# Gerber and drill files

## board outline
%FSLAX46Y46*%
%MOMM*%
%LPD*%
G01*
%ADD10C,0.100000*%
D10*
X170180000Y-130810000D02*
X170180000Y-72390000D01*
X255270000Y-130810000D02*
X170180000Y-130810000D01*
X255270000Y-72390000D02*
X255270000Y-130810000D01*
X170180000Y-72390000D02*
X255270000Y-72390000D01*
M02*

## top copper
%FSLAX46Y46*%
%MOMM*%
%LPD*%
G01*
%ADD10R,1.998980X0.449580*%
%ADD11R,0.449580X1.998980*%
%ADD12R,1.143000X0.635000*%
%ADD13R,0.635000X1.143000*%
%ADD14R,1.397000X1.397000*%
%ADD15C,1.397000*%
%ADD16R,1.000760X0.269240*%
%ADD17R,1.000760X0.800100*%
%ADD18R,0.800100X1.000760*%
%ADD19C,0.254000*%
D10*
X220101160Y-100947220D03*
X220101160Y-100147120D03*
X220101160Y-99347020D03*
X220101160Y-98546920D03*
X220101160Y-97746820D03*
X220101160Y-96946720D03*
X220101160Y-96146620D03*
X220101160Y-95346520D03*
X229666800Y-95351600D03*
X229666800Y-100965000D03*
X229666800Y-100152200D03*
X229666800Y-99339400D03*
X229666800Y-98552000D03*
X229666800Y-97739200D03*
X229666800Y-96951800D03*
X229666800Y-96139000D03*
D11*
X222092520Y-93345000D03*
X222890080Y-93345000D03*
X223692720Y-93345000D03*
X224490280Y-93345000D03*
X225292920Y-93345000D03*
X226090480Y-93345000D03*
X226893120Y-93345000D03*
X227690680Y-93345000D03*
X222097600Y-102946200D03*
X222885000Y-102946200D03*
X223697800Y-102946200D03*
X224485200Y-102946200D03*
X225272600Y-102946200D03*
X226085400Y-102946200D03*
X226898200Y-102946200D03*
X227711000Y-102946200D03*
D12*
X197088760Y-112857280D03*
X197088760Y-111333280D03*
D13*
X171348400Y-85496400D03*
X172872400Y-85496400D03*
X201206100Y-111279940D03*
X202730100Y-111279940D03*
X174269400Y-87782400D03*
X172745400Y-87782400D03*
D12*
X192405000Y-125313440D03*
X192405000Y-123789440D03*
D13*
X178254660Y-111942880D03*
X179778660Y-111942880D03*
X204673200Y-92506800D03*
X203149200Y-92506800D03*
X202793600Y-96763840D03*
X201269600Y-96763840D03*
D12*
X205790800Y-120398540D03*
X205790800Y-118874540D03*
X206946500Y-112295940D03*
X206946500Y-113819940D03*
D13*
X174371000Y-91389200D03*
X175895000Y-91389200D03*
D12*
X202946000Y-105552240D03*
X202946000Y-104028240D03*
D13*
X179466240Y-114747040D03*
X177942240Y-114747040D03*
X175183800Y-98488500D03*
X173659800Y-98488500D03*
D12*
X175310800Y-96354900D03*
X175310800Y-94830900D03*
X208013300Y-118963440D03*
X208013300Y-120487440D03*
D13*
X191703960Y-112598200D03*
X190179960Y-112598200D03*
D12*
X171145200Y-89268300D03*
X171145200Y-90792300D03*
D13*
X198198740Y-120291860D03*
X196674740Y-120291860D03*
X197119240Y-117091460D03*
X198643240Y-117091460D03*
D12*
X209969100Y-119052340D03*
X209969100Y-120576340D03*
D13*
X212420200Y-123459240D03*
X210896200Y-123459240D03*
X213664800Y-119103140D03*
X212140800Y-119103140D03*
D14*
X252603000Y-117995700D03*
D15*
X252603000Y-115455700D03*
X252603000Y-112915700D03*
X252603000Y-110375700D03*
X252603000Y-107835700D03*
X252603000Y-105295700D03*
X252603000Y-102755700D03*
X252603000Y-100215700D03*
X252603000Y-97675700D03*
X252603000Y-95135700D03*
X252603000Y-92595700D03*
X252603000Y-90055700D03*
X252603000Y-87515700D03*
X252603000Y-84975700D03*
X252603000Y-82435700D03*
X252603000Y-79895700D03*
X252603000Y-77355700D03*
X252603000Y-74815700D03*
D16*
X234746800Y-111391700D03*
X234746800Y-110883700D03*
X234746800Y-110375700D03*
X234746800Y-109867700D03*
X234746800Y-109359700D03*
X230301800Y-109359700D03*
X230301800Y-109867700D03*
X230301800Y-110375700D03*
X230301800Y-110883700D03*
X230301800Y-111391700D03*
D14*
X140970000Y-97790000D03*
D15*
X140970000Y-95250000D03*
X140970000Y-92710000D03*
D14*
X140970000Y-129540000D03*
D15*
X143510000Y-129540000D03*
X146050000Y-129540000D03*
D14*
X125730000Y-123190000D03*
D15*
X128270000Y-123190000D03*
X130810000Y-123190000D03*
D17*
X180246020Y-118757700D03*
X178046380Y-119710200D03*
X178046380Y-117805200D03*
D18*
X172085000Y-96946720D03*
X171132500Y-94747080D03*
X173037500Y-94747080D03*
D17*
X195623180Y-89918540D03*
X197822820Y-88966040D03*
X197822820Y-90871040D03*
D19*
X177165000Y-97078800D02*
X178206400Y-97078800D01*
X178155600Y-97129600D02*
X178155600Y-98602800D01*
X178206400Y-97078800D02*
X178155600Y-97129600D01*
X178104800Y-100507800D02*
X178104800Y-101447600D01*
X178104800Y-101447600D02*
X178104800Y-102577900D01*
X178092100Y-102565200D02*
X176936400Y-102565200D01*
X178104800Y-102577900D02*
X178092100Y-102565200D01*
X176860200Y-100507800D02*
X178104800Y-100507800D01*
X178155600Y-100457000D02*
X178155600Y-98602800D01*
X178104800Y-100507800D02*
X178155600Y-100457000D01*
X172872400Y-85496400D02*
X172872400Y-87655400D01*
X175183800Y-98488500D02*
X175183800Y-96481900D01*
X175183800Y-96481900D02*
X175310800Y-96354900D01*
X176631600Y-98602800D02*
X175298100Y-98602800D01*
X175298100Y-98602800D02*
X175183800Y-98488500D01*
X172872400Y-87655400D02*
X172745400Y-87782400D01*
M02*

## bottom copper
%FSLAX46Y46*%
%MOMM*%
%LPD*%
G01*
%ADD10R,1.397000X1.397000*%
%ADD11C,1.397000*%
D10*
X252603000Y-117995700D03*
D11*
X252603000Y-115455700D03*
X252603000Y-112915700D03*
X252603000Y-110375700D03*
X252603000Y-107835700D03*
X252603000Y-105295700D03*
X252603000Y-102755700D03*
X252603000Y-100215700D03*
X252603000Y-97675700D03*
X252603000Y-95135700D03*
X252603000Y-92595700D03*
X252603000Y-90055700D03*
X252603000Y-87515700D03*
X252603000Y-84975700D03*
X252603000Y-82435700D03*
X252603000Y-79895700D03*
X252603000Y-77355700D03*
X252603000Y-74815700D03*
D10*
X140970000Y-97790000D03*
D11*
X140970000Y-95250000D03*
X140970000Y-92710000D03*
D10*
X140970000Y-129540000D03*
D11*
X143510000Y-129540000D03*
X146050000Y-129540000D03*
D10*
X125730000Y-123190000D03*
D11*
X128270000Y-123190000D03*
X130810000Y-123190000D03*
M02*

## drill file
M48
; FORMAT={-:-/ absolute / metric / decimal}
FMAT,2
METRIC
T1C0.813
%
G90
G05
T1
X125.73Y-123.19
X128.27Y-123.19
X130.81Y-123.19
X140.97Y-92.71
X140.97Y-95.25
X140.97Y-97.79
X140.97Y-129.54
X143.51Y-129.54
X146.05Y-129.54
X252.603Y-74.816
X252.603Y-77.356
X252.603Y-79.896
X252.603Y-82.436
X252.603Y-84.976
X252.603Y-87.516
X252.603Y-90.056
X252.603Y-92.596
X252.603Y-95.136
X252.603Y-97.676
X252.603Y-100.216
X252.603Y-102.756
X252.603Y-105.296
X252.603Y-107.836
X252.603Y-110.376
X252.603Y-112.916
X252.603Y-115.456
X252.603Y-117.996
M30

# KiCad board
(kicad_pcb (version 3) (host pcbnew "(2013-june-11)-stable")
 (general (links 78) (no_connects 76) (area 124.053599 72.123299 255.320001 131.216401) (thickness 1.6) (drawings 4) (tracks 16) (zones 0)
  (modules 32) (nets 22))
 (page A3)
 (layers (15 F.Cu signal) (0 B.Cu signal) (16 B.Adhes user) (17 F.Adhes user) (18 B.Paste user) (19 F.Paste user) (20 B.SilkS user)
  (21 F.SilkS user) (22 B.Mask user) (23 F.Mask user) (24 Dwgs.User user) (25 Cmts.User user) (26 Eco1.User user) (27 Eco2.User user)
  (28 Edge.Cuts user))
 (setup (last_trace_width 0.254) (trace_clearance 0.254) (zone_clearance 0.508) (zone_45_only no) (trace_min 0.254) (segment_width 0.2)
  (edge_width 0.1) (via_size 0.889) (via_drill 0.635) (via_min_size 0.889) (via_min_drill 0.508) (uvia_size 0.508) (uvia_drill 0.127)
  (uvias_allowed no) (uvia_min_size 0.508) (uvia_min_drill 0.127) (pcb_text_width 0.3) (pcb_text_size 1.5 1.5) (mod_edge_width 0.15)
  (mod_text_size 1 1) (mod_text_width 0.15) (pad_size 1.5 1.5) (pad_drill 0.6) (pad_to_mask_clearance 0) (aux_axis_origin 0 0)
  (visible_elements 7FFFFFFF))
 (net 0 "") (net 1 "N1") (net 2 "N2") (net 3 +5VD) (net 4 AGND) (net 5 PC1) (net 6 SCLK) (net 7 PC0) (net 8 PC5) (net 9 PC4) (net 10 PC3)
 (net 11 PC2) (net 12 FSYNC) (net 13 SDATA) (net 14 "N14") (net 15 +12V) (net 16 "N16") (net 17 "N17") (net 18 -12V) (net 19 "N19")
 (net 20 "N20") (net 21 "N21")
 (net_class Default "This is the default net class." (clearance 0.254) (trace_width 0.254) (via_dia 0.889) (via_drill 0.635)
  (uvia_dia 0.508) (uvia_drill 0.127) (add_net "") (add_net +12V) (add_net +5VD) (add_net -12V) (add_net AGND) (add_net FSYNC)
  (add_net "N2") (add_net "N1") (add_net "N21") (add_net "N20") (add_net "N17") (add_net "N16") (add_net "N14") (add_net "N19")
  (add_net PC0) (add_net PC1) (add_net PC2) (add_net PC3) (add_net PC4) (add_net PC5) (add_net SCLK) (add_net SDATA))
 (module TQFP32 (layer F.Cu) (at 224.917 98.171)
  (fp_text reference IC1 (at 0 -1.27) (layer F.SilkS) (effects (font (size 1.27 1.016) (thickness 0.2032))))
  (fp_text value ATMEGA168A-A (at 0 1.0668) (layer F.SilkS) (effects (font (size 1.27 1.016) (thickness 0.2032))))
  (pad 8 smd rect (at -4.81584 2.77622) (size 1.99898 0.44958) (layers F.Cu F.Paste F.Mask) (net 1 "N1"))
  (pad 7 smd rect (at -4.81584 1.97612) (size 1.99898 0.44958) (layers F.Cu F.Paste F.Mask) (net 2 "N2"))
  (pad 6 smd rect (at -4.81584 1.17602) (size 1.99898 0.44958) (layers F.Cu F.Paste F.Mask) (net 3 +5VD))
  (pad 5 smd rect (at -4.81584 0.37592) (size 1.99898 0.44958) (layers F.Cu F.Paste F.Mask) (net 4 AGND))
  (pad 4 smd rect (at -4.81584 -0.42418) (size 1.99898 0.44958) (layers F.Cu F.Paste F.Mask) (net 3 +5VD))
  (pad 3 smd rect (at -4.81584 -1.22428) (size 1.99898 0.44958) (layers F.Cu F.Paste F.Mask) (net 4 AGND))
  (pad 2 smd rect (at -4.81584 -2.02438) (size 1.99898 0.44958) (layers F.Cu F.Paste F.Mask))
  (pad 1 smd rect (at -4.81584 -2.82448) (size 1.99898 0.44958) (layers F.Cu F.Paste F.Mask))
  (pad 24 smd rect (at 4.7498 -2.8194) (size 1.99898 0.44958) (layers F.Cu F.Paste F.Mask) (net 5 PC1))
  (pad 17 smd rect (at 4.7498 2.794) (size 1.99898 0.44958) (layers F.Cu F.Paste F.Mask) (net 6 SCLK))
  (pad 18 smd rect (at 4.7498 1.9812) (size 1.99898 0.44958) (layers F.Cu F.Paste F.Mask) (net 3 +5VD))
  (pad 19 smd rect (at 4.7498 1.1684) (size 1.99898 0.44958) (layers F.Cu F.Paste F.Mask))
  (pad 20 smd rect (at 4.7498 0.381) (size 1.99898 0.44958) (layers F.Cu F.Paste F.Mask))
  (pad 21 smd rect (at 4.7498 -0.4318) (size 1.99898 0.44958) (layers F.Cu F.Paste F.Mask) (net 4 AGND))
  (pad 22 smd rect (at 4.7498 -1.2192) (size 1.99898 0.44958) (layers F.Cu F.Paste F.Mask))
  (pad 23 smd rect (at 4.7498 -2.032) (size 1.99898 0.44958) (layers F.Cu F.Paste F.Mask) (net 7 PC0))
  (pad 32 smd rect (at -2.82448 -4.826) (size 0.44958 1.99898) (layers F.Cu F.Paste F.Mask))
  (pad 31 smd rect (at -2.02692 -4.826) (size 0.44958 1.99898) (layers F.Cu F.Paste F.Mask))
  (pad 30 smd rect (at -1.22428 -4.826) (size 0.44958 1.99898) (layers F.Cu F.Paste F.Mask))
  (pad 29 smd rect (at -0.42672 -4.826) (size 0.44958 1.99898) (layers F.Cu F.Paste F.Mask))
  (pad 28 smd rect (at 0.37592 -4.826) (size 0.44958 1.99898) (layers F.Cu F.Paste F.Mask) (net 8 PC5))
  (pad 27 smd rect (at 1.17348 -4.826) (size 0.44958 1.99898) (layers F.Cu F.Paste F.Mask) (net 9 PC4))
  (pad 26 smd rect (at 1.97612 -4.826) (size 0.44958 1.99898) (layers F.Cu F.Paste F.Mask) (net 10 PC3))
  (pad 25 smd rect (at 2.77368 -4.826) (size 0.44958 1.99898) (layers F.Cu F.Paste F.Mask) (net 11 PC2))
  (pad 9 smd rect (at -2.8194 4.7752) (size 0.44958 1.99898) (layers F.Cu F.Paste F.Mask))
  (pad 10 smd rect (at -2.032 4.7752) (size 0.44958 1.99898) (layers F.Cu F.Paste F.Mask))
  (pad 11 smd rect (at -1.2192 4.7752) (size 0.44958 1.99898) (layers F.Cu F.Paste F.Mask))
  (pad 12 smd rect (at -0.4318 4.7752) (size 0.44958 1.99898) (layers F.Cu F.Paste F.Mask))
  (pad 13 smd rect (at 0.3556 4.7752) (size 0.44958 1.99898) (layers F.Cu F.Paste F.Mask))
  (pad 14 smd rect (at 1.1684 4.7752) (size 0.44958 1.99898) (layers F.Cu F.Paste F.Mask))
  (pad 15 smd rect (at 1.9812 4.7752) (size 0.44958 1.99898) (layers F.Cu F.Paste F.Mask) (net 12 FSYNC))
  (pad 16 smd rect (at 2.794 4.7752) (size 0.44958 1.99898) (layers F.Cu F.Paste F.Mask) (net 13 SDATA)))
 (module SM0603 (layer F.Cu) (at 197.08876 112.09528 90)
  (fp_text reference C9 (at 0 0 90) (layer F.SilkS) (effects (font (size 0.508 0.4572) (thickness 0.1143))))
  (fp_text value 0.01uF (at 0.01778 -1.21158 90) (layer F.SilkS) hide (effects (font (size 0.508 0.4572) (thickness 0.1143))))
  (pad 1 smd rect (at -0.762 0 90) (size 0.635 1.143) (layers F.Cu F.Paste F.Mask) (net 4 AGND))
  (pad 2 smd rect (at 0.762 0 90) (size 0.635 1.143) (layers F.Cu F.Paste F.Mask) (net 3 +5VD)))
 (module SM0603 (layer F.Cu) (at 172.1104 85.4964)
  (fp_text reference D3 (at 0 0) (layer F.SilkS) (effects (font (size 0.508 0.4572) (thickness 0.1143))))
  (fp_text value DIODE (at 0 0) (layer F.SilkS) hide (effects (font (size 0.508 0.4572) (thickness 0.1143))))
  (pad 1 smd rect (at -0.762 0) (size 0.635 1.143) (layers F.Cu F.Paste F.Mask) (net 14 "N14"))
  (pad 2 smd rect (at 0.762 0) (size 0.635 1.143) (layers F.Cu F.Paste F.Mask) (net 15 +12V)))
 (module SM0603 (layer F.Cu) (at 201.9681 111.27994)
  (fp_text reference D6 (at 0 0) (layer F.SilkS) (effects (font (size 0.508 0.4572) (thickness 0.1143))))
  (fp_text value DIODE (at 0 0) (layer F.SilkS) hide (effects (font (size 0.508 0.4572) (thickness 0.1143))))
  (pad 1 smd rect (at -0.762 0) (size 0.635 1.143) (layers F.Cu F.Paste F.Mask) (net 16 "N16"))
  (pad 2 smd rect (at 0.762 0) (size 0.635 1.143) (layers F.Cu F.Paste F.Mask) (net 3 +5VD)))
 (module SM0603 (layer F.Cu) (at 173.5074 87.7824 180)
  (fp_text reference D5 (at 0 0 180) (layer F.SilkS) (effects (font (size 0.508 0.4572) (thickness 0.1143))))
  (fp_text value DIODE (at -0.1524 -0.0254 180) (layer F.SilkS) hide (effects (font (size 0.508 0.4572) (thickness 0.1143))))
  (pad 1 smd rect (at -0.762 0 180) (size 0.635 1.143) (layers F.Cu F.Paste F.Mask) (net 3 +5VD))
  (pad 2 smd rect (at 0.762 0 180) (size 0.635 1.143) (layers F.Cu F.Paste F.Mask) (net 15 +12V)))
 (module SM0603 (layer F.Cu) (at 192.405 124.55144 90)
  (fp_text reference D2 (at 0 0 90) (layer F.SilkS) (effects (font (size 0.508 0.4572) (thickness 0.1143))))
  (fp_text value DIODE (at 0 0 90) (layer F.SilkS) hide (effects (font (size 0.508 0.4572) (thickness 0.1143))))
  (pad 1 smd rect (at -0.762 0 90) (size 0.635 1.143) (layers F.Cu F.Paste F.Mask))
  (pad 2 smd rect (at 0.762 0 90) (size 0.635 1.143) (layers F.Cu F.Paste F.Mask)))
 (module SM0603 (layer F.Cu) (at 179.01666 111.94288)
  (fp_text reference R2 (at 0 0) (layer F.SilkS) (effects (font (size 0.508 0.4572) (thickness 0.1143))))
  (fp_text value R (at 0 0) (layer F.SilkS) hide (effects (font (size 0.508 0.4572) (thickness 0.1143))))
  (pad 1 smd rect (at -0.762 0) (size 0.635 1.143) (layers F.Cu F.Paste F.Mask) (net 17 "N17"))
  (pad 2 smd rect (at 0.762 0) (size 0.635 1.143) (layers F.Cu F.Paste F.Mask) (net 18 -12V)))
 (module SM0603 (layer F.Cu) (at 203.9112 92.5068 180)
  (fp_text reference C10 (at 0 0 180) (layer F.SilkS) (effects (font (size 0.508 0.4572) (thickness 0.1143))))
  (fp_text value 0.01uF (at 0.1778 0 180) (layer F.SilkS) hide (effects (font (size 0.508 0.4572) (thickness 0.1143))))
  (pad 1 smd rect (at -0.762 0 180) (size 0.635 1.143) (layers F.Cu F.Paste F.Mask) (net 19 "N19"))
  (pad 2 smd rect (at 0.762 0 180) (size 0.635 1.143) (layers F.Cu F.Paste F.Mask) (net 3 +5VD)))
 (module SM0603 (layer F.Cu) (at 202.0316 96.76384 180)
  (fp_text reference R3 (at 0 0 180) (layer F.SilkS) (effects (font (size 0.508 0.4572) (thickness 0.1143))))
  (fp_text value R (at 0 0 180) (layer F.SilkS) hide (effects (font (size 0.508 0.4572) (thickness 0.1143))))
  (pad 1 smd rect (at -0.762 0 180) (size 0.635 1.143) (layers F.Cu F.Paste F.Mask) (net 3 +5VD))
  (pad 2 smd rect (at 0.762 0 180) (size 0.635 1.143) (layers F.Cu F.Paste F.Mask) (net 16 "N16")))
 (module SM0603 (layer F.Cu) (at 205.7908 119.63654 90)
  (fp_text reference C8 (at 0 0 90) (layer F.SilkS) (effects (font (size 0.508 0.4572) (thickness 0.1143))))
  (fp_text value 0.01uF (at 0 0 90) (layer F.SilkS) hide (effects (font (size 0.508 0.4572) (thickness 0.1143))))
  (pad 1 smd rect (at -0.762 0 90) (size 0.635 1.143) (layers F.Cu F.Paste F.Mask) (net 4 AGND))
  (pad 2 smd rect (at 0.762 0 90) (size 0.635 1.143) (layers F.Cu F.Paste F.Mask) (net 3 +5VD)))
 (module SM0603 (layer F.Cu) (at 206.9465 113.05794 270)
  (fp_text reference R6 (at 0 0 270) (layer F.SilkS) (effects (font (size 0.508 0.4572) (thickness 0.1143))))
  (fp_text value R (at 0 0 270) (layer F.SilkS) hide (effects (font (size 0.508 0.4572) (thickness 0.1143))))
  (pad 1 smd rect (at -0.762 0 270) (size 0.635 1.143) (layers F.Cu F.Paste F.Mask) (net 3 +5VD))
  (pad 2 smd rect (at 0.762 0 270) (size 0.635 1.143) (layers F.Cu F.Paste F.Mask) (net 12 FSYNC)))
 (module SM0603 (layer F.Cu) (at 175.133 91.3892)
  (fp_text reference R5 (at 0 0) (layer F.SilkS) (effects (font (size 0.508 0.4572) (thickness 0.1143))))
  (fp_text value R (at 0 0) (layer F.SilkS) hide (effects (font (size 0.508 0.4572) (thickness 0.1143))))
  (pad 1 smd rect (at -0.762 0) (size 0.635 1.143) (layers F.Cu F.Paste F.Mask) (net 3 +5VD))
  (pad 2 smd rect (at 0.762 0) (size 0.635 1.143) (layers F.Cu F.Paste F.Mask) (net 13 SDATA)))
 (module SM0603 (layer F.Cu) (at 202.946 104.79024 90)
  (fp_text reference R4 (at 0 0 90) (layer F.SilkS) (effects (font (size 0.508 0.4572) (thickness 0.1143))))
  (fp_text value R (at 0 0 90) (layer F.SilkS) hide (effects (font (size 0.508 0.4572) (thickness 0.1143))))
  (pad 1 smd rect (at -0.762 0 90) (size 0.635 1.143) (layers F.Cu F.Paste F.Mask) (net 3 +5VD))
  (pad 2 smd rect (at 0.762 0 90) (size 0.635 1.143) (layers F.Cu F.Paste F.Mask) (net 6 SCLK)))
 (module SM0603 (layer F.Cu) (at 178.70424 114.74704 180)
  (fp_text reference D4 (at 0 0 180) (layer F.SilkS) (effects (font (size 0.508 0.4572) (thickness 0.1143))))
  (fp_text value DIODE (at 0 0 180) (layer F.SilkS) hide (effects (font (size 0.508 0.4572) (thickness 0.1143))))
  (pad 1 smd rect (at -0.762 0 180) (size 0.635 1.143) (layers F.Cu F.Paste F.Mask) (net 18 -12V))
  (pad 2 smd rect (at 0.762 0 180) (size 0.635 1.143) (layers F.Cu F.Paste F.Mask) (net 17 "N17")))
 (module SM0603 (layer F.Cu) (at 174.4218 98.4885 180)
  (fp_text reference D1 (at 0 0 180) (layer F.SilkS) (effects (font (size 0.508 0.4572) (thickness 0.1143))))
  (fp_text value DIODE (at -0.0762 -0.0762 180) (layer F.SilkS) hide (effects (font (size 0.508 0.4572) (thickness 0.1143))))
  (pad 1 smd rect (at -0.762 0 180) (size 0.635 1.143) (layers F.Cu F.Paste F.Mask) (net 15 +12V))
  (pad 2 smd rect (at 0.762 0 180) (size 0.635 1.143) (layers F.Cu F.Paste F.Mask) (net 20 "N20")))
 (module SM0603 (layer F.Cu) (at 175.3108 95.5929 90)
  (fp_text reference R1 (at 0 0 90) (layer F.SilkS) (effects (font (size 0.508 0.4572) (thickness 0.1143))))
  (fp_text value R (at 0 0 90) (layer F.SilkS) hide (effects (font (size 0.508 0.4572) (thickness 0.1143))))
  (pad 1 smd rect (at -0.762 0 90) (size 0.635 1.143) (layers F.Cu F.Paste F.Mask) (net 15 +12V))
  (pad 2 smd rect (at 0.762 0 90) (size 0.635 1.143) (layers F.Cu F.Paste F.Mask) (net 14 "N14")))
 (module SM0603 (layer F.Cu) (at 208.0133 119.72544 270)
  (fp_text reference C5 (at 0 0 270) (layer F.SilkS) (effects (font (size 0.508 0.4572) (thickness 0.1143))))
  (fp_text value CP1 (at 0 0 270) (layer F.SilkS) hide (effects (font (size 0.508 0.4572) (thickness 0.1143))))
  (pad 1 smd rect (at -0.762 0 270) (size 0.635 1.143) (layers F.Cu F.Paste F.Mask) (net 3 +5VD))
  (pad 2 smd rect (at 0.762 0 270) (size 0.635 1.143) (layers F.Cu F.Paste F.Mask) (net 4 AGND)))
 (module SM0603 (layer F.Cu) (at 190.94196 112.5982 180)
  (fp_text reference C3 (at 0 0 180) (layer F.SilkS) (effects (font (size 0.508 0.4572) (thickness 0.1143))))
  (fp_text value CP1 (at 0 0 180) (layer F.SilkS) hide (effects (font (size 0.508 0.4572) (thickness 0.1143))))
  (pad 1 smd rect (at -0.762 0 180) (size 0.635 1.143) (layers F.Cu F.Paste F.Mask) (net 15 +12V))
  (pad 2 smd rect (at 0.762 0 180) (size 0.635 1.143) (layers F.Cu F.Paste F.Mask) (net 4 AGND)))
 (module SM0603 (layer F.Cu) (at 171.1452 90.0303 270)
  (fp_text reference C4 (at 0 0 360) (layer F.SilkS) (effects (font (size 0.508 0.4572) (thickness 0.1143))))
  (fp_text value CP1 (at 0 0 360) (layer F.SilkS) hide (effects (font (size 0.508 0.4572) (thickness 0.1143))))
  (pad 1 smd rect (at -0.762 0 270) (size 0.635 1.143) (layers F.Cu F.Paste F.Mask) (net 4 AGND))
  (pad 2 smd rect (at 0.762 0 270) (size 0.635 1.143) (layers F.Cu F.Paste F.Mask) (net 18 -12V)))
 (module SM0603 (layer F.Cu) (at 197.43674 120.29186 180)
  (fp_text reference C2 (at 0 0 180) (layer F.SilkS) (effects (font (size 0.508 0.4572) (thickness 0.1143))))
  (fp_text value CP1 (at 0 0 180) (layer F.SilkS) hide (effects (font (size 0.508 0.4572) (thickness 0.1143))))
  (pad 1 smd rect (at -0.762 0 180) (size 0.635 1.143) (layers F.Cu F.Paste F.Mask) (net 4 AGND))
  (pad 2 smd rect (at 0.762 0 180) (size 0.635 1.143) (layers F.Cu F.Paste F.Mask) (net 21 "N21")))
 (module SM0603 (layer F.Cu) (at 197.88124 117.09146)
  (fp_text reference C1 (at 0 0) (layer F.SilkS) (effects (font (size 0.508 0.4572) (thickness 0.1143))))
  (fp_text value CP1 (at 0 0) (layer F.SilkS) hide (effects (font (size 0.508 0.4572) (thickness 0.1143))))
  (pad 1 smd rect (at -0.762 0) (size 0.635 1.143) (layers F.Cu F.Paste F.Mask) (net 20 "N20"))
  (pad 2 smd rect (at 0.762 0) (size 0.635 1.143) (layers F.Cu F.Paste F.Mask) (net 4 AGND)))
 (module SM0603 (layer F.Cu) (at 209.9691 119.81434 270)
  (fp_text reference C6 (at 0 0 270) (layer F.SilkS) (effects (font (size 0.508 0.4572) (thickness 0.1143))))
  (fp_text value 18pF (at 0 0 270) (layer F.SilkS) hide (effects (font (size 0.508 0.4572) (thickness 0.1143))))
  (pad 1 smd rect (at -0.762 0 270) (size 0.635 1.143) (layers F.Cu F.Paste F.Mask) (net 2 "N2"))
  (pad 2 smd rect (at 0.762 0 270) (size 0.635 1.143) (layers F.Cu F.Paste F.Mask) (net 4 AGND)))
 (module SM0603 (layer F.Cu) (at 211.6582 123.45924 180)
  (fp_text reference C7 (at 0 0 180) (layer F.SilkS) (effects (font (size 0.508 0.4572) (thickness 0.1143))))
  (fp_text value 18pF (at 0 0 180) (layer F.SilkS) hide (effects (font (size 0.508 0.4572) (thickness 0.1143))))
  (pad 1 smd rect (at -0.762 0 180) (size 0.635 1.143) (layers F.Cu F.Paste F.Mask) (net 1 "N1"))
  (pad 2 smd rect (at 0.762 0 180) (size 0.635 1.143) (layers F.Cu F.Paste F.Mask) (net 4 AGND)))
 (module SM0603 (layer F.Cu) (at 212.9028 119.10314 180)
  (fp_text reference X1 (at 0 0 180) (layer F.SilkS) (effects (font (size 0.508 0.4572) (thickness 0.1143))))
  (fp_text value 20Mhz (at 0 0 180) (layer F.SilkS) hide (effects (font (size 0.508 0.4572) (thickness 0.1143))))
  (pad 1 smd rect (at -0.762 0 180) (size 0.635 1.143) (layers F.Cu F.Paste F.Mask) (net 1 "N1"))
  (pad 2 smd rect (at 0.762 0 180) (size 0.635 1.143) (layers F.Cu F.Paste F.Mask) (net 2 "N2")))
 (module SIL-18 (layer F.Cu) (at 252.603 96.4057 90)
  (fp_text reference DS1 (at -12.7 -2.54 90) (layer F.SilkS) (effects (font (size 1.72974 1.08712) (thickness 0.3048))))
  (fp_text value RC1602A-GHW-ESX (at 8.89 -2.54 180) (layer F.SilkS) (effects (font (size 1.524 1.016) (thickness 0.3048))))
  (pad 1 thru_hole rect (at -21.59 0 90) (size 1.397 1.397) (drill 0.8128) (layers *.Cu *.Mask F.SilkS) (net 4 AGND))
  (pad 2 thru_hole circle (at -19.05 0 90) (size 1.397 1.397) (drill 0.8128) (layers *.Cu *.Mask F.SilkS) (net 3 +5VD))
  (pad 3 thru_hole circle (at -16.51 0 90) (size 1.397 1.397) (drill 0.8128) (layers *.Cu *.Mask F.SilkS) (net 3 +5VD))
  (pad 4 thru_hole circle (at -13.97 0 90) (size 1.397 1.397) (drill 0.8128) (layers *.Cu *.Mask F.SilkS) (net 9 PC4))
  (pad 5 thru_hole circle (at -11.43 0 90) (size 1.397 1.397) (drill 0.8128) (layers *.Cu *.Mask F.SilkS) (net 4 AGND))
  (pad 6 thru_hole circle (at -8.89 0 90) (size 1.397 1.397) (drill 0.8128) (layers *.Cu *.Mask F.SilkS) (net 8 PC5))
  (pad 7 thru_hole circle (at -6.35 0 90) (size 1.397 1.397) (drill 0.8128) (layers *.Cu *.Mask F.SilkS))
  (pad 8 thru_hole circle (at -3.81 0 90) (size 1.397 1.397) (drill 0.8128) (layers *.Cu *.Mask F.SilkS))
  (pad 9 thru_hole circle (at -1.27 0 90) (size 1.397 1.397) (drill 0.8128) (layers *.Cu *.Mask F.SilkS))
  (pad 10 thru_hole circle (at 1.27 0 90) (size 1.397 1.397) (drill 0.8128) (layers *.Cu *.Mask F.SilkS))
  (pad 11 thru_hole circle (at 3.81 0 90) (size 1.397 1.397) (drill 0.8128) (layers *.Cu *.Mask F.SilkS) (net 7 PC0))
  (pad 12 thru_hole circle (at 6.35 0 90) (size 1.397 1.397) (drill 0.8128) (layers *.Cu *.Mask F.SilkS) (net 5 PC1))
  (pad 13 thru_hole circle (at 8.89 0 90) (size 1.397 1.397) (drill 0.8128) (layers *.Cu *.Mask F.SilkS) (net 11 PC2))
  (pad 14 thru_hole circle (at 11.43 0 90) (size 1.397 1.397) (drill 0.8128) (layers *.Cu *.Mask F.SilkS) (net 10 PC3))
  (pad 15 thru_hole circle (at 13.97 0 90) (size 1.397 1.397) (drill 0.8128) (layers *.Cu *.Mask F.SilkS) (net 3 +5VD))
  (pad 16 thru_hole circle (at 16.51 0 90) (size 1.397 1.397) (drill 0.8128) (layers *.Cu *.Mask F.SilkS) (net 4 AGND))
  (pad 17 thru_hole circle (at 19.05 0 90) (size 1.397 1.397) (drill 0.8128) (layers *.Cu *.Mask F.SilkS))
  (pad 18 thru_hole circle (at 21.59 0 90) (size 1.397 1.397) (drill 0.8128) (layers *.Cu *.Mask F.SilkS)))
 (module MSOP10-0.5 (layer F.Cu) (at 232.5243 110.3757 90)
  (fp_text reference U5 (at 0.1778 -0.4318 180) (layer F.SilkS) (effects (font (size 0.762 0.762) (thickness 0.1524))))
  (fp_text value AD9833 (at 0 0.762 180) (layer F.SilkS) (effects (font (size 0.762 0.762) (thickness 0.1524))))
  (pad 1 smd rect (at -1.016 2.2225 90) (size 0.26924 1.00076) (layers F.Cu F.Paste F.Mask) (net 19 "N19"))
  (pad 2 smd rect (at -0.508 2.2225 90) (size 0.26924 1.00076) (layers F.Cu F.Paste F.Mask) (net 3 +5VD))
  (pad 3 smd rect (at 0 2.2225 90) (size 0.26924 1.00076) (layers F.Cu F.Paste F.Mask) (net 3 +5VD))
  (pad 4 smd rect (at 0.508 2.2225 90) (size 0.26924 1.00076) (layers F.Cu F.Paste F.Mask) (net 4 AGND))
  (pad 5 smd rect (at 1.016 2.2225 90) (size 0.26924 1.00076) (layers F.Cu F.Paste F.Mask))
  (pad 6 smd rect (at 1.016 -2.2225 90) (size 0.26924 1.00076) (layers F.Cu F.Paste F.Mask) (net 13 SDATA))
  (pad 7 smd rect (at 0.508 -2.2225 90) (size 0.26924 1.00076) (layers F.Cu F.Paste F.Mask) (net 6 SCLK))
  (pad 8 smd rect (at 0 -2.2225 90) (size 0.26924 1.00076) (layers F.Cu F.Paste F.Mask) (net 12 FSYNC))
  (pad 9 smd rect (at -0.508 -2.2225 90) (size 0.26924 1.00076) (layers F.Cu F.Paste F.Mask) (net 4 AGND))
  (pad 10 smd rect (at -1.016 -2.2225 90) (size 0.26924 1.00076) (layers F.Cu F.Paste F.Mask)))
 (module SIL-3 (layer F.Cu) (at 140.97 95.25 90)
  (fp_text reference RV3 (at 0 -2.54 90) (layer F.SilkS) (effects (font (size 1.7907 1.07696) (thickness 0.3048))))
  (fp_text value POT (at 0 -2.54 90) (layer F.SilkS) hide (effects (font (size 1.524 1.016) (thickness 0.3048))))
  (pad 1 thru_hole rect (at -2.54 0 90) (size 1.397 1.397) (drill 0.8128) (layers *.Cu *.Mask F.SilkS) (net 16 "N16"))
  (pad 2 thru_hole circle (at 0 0 90) (size 1.397 1.397) (drill 0.8128) (layers *.Cu *.Mask F.SilkS) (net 16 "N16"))
  (pad 3 thru_hole circle (at 2.54 0 90) (size 1.397 1.397) (drill 0.8128) (layers *.Cu *.Mask F.SilkS) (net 4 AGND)))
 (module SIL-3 (layer F.Cu) (at 143.51 129.54)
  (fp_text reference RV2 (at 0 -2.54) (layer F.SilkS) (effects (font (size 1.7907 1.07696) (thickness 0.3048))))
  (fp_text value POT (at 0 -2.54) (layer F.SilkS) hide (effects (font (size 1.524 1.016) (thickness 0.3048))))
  (pad 1 thru_hole rect (at -2.54 0) (size 1.397 1.397) (drill 0.8128) (layers *.Cu *.Mask F.SilkS) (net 4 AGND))
  (pad 2 thru_hole circle (at 0 0) (size 1.397 1.397) (drill 0.8128) (layers *.Cu *.Mask F.SilkS) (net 17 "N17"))
  (pad 3 thru_hole circle (at 2.54 0) (size 1.397 1.397) (drill 0.8128) (layers *.Cu *.Mask F.SilkS) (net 17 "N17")))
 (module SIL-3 (layer F.Cu) (at 128.27 123.19)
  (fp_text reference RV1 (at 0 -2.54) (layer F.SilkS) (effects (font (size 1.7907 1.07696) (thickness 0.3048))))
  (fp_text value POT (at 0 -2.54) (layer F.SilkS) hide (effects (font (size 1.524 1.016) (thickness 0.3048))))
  (pad 1 thru_hole rect (at -2.54 0) (size 1.397 1.397) (drill 0.8128) (layers *.Cu *.Mask F.SilkS) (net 14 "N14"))
  (pad 2 thru_hole circle (at 0 0) (size 1.397 1.397) (drill 0.8128) (layers *.Cu *.Mask F.SilkS) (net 14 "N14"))
  (pad 3 thru_hole circle (at 2.54 0) (size 1.397 1.397) (drill 0.8128) (layers *.Cu *.Mask F.SilkS) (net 4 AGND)))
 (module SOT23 (layer F.Cu) (at 179.1462 118.7577 270)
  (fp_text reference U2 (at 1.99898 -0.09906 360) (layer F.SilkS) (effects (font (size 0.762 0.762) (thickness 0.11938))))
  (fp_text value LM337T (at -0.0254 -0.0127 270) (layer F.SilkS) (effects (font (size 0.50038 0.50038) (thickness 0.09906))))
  (pad 3 smd rect (at 0 -1.09982 270) (size 0.8001 1.00076) (layers F.Cu F.Paste F.Mask) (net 18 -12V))
  (pad 2 smd rect (at 0.9525 1.09982 270) (size 0.8001 1.00076) (layers F.Cu F.Paste F.Mask) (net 21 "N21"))
  (pad 1 smd rect (at -0.9525 1.09982 270) (size 0.8001 1.00076) (layers F.Cu F.Paste F.Mask) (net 17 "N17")))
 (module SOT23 (layer F.Cu) (at 172.085 95.8469 180)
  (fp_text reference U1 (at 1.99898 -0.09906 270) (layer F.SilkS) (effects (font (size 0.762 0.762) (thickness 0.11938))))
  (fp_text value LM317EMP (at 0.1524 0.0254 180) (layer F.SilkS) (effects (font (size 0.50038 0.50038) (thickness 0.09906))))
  (pad 3 smd rect (at 0 -1.09982 180) (size 0.8001 1.00076) (layers F.Cu F.Paste F.Mask) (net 20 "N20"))
  (pad 2 smd rect (at 0.9525 1.09982 180) (size 0.8001 1.00076) (layers F.Cu F.Paste F.Mask) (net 15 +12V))
  (pad 1 smd rect (at -0.9525 1.09982 180) (size 0.8001 1.00076) (layers F.Cu F.Paste F.Mask) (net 14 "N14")))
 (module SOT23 (layer F.Cu) (at 196.723 89.91854 90)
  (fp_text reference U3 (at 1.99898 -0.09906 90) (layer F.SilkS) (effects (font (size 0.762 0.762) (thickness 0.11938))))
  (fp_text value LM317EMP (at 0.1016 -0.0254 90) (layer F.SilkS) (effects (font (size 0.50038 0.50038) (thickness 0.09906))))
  (pad 3 smd rect (at 0 -1.09982 90) (size 0.8001 1.00076) (layers F.Cu F.Paste F.Mask) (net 15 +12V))
  (pad 2 smd rect (at 0.9525 1.09982 90) (size 0.8001 1.00076) (layers F.Cu F.Paste F.Mask) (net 3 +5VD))
  (pad 1 smd rect (at -0.9525 1.09982 90) (size 0.8001 1.00076) (layers F.Cu F.Paste F.Mask) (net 16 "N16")))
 (gr_line (start 170.18 130.81) (end 170.18 72.39) (angle 90) (layer Edge.Cuts) (width 0.1))
 (gr_line (start 255.27 130.81) (end 170.18 130.81) (angle 90) (layer Edge.Cuts) (width 0.1))
 (gr_line (start 255.27 72.39) (end 255.27 130.81) (angle 90) (layer Edge.Cuts) (width 0.1))
 (gr_line (start 170.18 72.39) (end 255.27 72.39) (angle 90) (layer Edge.Cuts) (width 0.1))
 (segment (start 177.165 97.0788) (end 178.2064 97.0788) (width 0.254) (layer F.Cu) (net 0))
 (segment (start 178.1556 97.1296) (end 178.1556 98.6028) (width 0.254) (layer F.Cu) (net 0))
 (segment (start 178.2064 97.0788) (end 178.1556 97.1296) (width 0.254) (layer F.Cu) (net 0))
 (segment (start 178.1048 100.5078) (end 178.1048 101.4476) (width 0.254) (layer F.Cu) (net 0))
 (segment (start 178.1048 101.4476) (end 178.1048 102.5779) (width 0.254) (layer F.Cu) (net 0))
 (segment (start 178.0921 102.5652) (end 176.9364 102.5652) (width 0.254) (layer F.Cu) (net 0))
 (segment (start 178.1048 102.5779) (end 178.0921 102.5652) (width 0.254) (layer F.Cu) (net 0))
 (segment (start 176.8602 100.5078) (end 178.1048 100.5078) (width 0.254) (layer F.Cu) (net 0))
 (segment (start 178.1556 100.457) (end 178.1556 98.6028) (width 0.254) (layer F.Cu) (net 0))
 (segment (start 178.1048 100.5078) (end 178.1556 100.457) (width 0.254) (layer F.Cu) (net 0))
 (segment (start 172.8724 85.4964) (end 172.8724 87.6554) (width 0.254) (layer F.Cu) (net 15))
 (segment (start 175.1838 98.4885) (end 175.1838 96.4819) (width 0.254) (layer F.Cu) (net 15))
 (segment (start 175.1838 96.4819) (end 175.3108 96.3549) (width 0.254) (layer F.Cu) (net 15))
 (segment (start 176.6316 98.6028) (end 175.2981 98.6028) (width 0.254) (layer F.Cu) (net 15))
 (segment (start 175.2981 98.6028) (end 175.1838 98.4885) (width 0.254) (layer F.Cu) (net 15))
 (segment (start 172.8724 87.6554) (end 172.7454 87.7824) (width 0.254) (layer F.Cu) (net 15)))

